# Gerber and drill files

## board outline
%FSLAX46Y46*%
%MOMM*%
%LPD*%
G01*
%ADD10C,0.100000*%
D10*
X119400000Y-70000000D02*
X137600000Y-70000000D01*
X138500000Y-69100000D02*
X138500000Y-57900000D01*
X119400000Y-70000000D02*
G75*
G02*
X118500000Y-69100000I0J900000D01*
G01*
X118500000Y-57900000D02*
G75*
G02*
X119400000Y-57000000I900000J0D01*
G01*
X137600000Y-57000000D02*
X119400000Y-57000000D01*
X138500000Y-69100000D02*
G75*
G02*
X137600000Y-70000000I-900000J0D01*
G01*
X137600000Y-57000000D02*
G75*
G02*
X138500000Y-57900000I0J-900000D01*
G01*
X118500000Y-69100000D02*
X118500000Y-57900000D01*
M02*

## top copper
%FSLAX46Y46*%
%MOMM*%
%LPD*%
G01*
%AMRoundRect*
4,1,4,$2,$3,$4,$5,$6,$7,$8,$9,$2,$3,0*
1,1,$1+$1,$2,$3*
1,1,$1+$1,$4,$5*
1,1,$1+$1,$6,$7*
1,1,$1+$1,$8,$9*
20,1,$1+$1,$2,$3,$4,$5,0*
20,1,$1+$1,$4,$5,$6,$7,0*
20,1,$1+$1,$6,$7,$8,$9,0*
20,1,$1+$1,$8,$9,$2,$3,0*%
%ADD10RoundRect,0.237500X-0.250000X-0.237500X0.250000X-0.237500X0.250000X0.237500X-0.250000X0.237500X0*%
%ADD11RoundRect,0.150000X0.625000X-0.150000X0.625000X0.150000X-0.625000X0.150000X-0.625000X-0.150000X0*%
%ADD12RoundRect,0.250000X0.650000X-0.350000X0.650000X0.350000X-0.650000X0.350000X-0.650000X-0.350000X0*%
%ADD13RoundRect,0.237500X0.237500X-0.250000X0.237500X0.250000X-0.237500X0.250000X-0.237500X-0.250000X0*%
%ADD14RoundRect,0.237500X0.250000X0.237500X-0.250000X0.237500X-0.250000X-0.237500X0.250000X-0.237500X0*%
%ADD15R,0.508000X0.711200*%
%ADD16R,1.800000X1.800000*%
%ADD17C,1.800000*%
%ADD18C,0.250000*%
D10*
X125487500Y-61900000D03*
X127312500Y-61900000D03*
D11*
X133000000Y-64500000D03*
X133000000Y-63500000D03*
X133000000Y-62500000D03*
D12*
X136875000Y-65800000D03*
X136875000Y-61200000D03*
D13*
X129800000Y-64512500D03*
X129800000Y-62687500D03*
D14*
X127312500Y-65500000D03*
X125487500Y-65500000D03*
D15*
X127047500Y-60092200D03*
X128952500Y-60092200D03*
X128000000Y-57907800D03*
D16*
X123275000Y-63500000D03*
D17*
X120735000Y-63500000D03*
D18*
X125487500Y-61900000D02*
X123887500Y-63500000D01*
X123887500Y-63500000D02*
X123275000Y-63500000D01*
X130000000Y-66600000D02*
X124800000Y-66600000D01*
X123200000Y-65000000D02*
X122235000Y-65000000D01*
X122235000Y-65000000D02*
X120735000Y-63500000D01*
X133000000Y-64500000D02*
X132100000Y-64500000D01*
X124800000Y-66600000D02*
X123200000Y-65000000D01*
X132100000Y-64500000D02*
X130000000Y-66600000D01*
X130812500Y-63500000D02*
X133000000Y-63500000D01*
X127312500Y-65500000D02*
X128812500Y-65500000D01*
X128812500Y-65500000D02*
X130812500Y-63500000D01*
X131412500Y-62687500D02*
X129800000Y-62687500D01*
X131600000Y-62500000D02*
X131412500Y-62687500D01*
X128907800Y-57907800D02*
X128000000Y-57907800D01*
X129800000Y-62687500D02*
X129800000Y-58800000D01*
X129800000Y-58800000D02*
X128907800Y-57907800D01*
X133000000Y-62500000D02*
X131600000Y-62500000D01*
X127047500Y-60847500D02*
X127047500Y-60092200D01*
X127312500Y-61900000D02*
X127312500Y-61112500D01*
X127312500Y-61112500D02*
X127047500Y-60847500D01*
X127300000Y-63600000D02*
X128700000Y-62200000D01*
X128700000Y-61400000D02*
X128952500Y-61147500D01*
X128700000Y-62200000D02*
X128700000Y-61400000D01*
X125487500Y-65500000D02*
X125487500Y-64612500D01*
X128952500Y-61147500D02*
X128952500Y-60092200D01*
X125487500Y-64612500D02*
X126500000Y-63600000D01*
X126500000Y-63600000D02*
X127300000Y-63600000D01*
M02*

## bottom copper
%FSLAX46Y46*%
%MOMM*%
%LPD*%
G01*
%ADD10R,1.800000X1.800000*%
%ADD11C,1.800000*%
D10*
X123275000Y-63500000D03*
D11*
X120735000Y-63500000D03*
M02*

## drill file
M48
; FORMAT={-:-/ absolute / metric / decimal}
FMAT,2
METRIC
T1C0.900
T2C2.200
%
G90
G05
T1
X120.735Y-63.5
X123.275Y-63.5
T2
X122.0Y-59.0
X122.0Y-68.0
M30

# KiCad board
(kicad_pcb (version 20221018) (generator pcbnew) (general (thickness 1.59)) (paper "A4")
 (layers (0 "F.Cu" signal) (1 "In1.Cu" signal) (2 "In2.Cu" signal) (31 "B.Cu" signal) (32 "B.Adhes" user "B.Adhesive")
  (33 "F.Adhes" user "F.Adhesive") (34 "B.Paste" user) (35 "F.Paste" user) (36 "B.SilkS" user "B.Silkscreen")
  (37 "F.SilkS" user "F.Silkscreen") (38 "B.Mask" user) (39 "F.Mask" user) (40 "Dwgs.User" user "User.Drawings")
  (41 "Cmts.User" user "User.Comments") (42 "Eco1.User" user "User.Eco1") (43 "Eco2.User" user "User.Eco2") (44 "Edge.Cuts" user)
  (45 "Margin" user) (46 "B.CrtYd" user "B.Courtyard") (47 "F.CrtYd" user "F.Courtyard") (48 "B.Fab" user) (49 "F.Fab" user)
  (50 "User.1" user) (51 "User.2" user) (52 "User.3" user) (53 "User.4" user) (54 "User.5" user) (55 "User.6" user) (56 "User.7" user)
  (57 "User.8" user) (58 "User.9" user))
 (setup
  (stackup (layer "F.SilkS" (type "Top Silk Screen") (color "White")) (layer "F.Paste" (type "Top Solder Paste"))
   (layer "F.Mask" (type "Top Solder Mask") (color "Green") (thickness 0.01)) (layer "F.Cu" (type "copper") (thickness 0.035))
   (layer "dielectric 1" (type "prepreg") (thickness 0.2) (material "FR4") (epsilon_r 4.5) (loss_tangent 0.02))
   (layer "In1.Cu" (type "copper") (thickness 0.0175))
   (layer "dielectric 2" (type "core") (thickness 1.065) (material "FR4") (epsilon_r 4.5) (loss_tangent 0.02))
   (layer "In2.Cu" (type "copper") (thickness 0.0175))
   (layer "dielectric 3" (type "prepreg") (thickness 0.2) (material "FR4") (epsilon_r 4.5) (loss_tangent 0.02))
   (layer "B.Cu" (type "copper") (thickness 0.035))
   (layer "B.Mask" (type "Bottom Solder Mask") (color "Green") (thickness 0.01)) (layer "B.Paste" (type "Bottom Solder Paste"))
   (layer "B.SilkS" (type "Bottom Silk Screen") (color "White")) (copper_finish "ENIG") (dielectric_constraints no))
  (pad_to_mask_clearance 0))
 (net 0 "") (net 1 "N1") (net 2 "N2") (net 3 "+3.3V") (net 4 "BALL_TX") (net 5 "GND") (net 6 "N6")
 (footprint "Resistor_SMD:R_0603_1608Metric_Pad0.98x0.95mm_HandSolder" (layer "F.Cu") (at 126.4 61.9)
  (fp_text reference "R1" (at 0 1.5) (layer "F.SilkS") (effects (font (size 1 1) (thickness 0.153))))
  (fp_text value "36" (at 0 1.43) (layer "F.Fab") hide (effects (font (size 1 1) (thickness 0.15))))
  (pad "1" smd roundrect (at -0.9125 0) (size 0.975 0.95) (layers "F.Cu" "F.Paste" "F.Mask") (roundrect_rratio 0.25) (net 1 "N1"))
  (pad "2" smd roundrect (at 0.9125 0) (size 0.975 0.95) (layers "F.Cu" "F.Paste" "F.Mask") (roundrect_rratio 0.25) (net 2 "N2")))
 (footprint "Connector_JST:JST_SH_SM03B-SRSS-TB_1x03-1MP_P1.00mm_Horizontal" (layer "F.Cu") (at 135 63.5 90)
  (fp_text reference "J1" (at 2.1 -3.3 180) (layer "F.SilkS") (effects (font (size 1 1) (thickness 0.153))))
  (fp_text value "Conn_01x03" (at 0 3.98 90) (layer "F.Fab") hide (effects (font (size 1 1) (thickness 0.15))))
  (pad "1" smd roundrect (at -1 -2 90) (size 0.6 1.55) (layers "F.Cu" "F.Paste" "F.Mask") (roundrect_rratio 0.25) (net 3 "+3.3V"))
  (pad "2" smd roundrect (at 0 -2 90) (size 0.6 1.55) (layers "F.Cu" "F.Paste" "F.Mask") (roundrect_rratio 0.25) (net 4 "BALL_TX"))
  (pad "3" smd roundrect (at 1 -2 90) (size 0.6 1.55) (layers "F.Cu" "F.Paste" "F.Mask") (roundrect_rratio 0.25) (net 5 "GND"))
  (pad "MP" smd roundrect (at -2.3 1.875 90) (size 1.2 1.8) (layers "F.Cu" "F.Paste" "F.Mask") (roundrect_rratio 0.208333))
  (pad "MP" smd roundrect (at 2.3 1.875 90) (size 1.2 1.8) (layers "F.Cu" "F.Paste" "F.Mask") (roundrect_rratio 0.208333)))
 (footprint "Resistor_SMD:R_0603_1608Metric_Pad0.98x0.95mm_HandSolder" (layer "F.Cu") (at 129.8 63.6 90)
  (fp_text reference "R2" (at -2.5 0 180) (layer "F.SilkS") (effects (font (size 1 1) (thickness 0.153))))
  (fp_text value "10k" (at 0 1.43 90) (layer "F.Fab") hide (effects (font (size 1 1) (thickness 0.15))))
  (pad "1" smd roundrect (at -0.9125 0 90) (size 0.975 0.95) (layers "F.Cu" "F.Paste" "F.Mask") (roundrect_rratio 0.25) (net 4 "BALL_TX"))
  (pad "2" smd roundrect (at 0.9125 0 90) (size 0.975 0.95) (layers "F.Cu" "F.Paste" "F.Mask") (roundrect_rratio 0.25) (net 5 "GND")))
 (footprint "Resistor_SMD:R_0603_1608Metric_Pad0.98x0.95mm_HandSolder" (layer "F.Cu") (at 126.4 65.5 180)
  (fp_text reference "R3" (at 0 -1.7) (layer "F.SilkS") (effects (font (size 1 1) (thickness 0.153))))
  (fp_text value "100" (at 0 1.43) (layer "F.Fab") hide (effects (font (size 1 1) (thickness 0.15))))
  (pad "1" smd roundrect (at -0.9125 0 180) (size 0.975 0.95) (layers "F.Cu" "F.Paste" "F.Mask") (roundrect_rratio 0.25) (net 4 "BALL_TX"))
  (pad "2" smd roundrect (at 0.9125 0 180) (size 0.975 0.95) (layers "F.Cu" "F.Paste" "F.Mask") (roundrect_rratio 0.25) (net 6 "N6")))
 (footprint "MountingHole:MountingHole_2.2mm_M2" (layer "F.Cu") (at 122 68 -90)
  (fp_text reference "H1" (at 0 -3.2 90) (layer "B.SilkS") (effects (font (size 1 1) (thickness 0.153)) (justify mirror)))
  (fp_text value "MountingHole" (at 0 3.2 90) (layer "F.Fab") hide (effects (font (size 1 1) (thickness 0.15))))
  (pad "" np_thru_hole circle (at 0 0 270) (size 2.2 2.2) (drill 2.2) (layers "*.Cu" "*.Mask")))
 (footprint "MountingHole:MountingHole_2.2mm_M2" (layer "F.Cu") (at 122 59 -90)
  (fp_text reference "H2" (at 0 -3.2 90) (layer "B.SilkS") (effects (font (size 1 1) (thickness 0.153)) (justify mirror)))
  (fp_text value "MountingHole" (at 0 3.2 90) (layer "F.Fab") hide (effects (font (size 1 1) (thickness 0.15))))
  (pad "" np_thru_hole circle (at 0 0 270) (size 2.2 2.2) (drill 2.2) (layers "*.Cu" "*.Mask")))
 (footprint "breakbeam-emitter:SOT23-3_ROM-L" (layer "F.Cu") (at 128 59)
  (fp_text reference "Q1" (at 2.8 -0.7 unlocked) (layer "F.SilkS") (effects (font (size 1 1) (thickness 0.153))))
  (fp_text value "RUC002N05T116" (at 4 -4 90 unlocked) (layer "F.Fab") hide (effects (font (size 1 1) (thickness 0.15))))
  (pad "1" smd rect (at -0.9525 1.0922) (size 0.508 0.7112) (layers "F.Cu" "F.Paste" "F.Mask") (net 2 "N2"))
  (pad "2" smd rect (at 0.9525 1.0922) (size 0.508 0.7112) (layers "F.Cu" "F.Paste" "F.Mask") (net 6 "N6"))
  (pad "3" smd rect (at 0 -1.0922) (size 0.508 0.7112) (layers "F.Cu" "F.Paste" "F.Mask") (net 5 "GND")))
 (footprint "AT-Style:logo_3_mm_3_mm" (layer "B.Cu") (at 135.5 60.5 180)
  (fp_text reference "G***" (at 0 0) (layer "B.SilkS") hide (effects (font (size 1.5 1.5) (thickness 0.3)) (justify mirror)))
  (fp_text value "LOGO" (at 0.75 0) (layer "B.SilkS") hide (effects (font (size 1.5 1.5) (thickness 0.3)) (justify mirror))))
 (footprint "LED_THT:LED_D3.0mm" (layer "B.Cu") (at 123.275 63.5 180)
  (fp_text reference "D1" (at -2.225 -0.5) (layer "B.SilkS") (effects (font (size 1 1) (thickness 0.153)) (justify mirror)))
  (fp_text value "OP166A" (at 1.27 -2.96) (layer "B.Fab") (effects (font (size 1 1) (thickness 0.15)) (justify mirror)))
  (pad "1" thru_hole rect (at 0 0 180) (size 1.8 1.8) (drill 0.9) (layers "*.Cu" "*.Mask") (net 1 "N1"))
  (pad "2" thru_hole circle (at 2.54 0 180) (size 1.8 1.8) (drill 0.9) (layers "*.Cu" "*.Mask") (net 3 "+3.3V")))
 (gr_line (start 119.4 70) (end 137.6 70) (stroke (width 0.1) (type default)) (layer "Edge.Cuts"))
 (gr_line (start 138.5 69.1) (end 138.5 57.9) (stroke (width 0.1) (type default)) (layer "Edge.Cuts"))
 (gr_arc (start 119.4 70) (mid 118.763604 69.736396) (end 118.5 69.1) (stroke (width 0.1) (type default)) (layer "Edge.Cuts"))
 (gr_arc (start 118.5 57.9) (mid 118.763604 57.263604) (end 119.4 57) (stroke (width 0.1) (type default)) (layer "Edge.Cuts"))
 (gr_line (start 137.6 57) (end 119.4 57) (stroke (width 0.1) (type default)) (layer "Edge.Cuts"))
 (gr_arc (start 138.5 69.1) (mid 138.236396 69.736396) (end 137.6 70) (stroke (width 0.1) (type default)) (layer "Edge.Cuts"))
 (gr_arc (start 137.6 57) (mid 138.236396 57.263604) (end 138.5 57.9) (stroke (width 0.1) (type default)) (layer "Edge.Cuts"))
 (gr_line (start 118.5 69.1) (end 118.5 57.9) (stroke (width 0.1) (type default)) (layer "Edge.Cuts"))
 (segment (start 125.4875 61.9) (end 123.8875 63.5) (width 0.25) (layer "F.Cu") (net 1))
 (segment (start 123.8875 63.5) (end 123.275 63.5) (width 0.25) (layer "F.Cu") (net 1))
 (segment (start 130 66.6) (end 124.8 66.6) (width 0.25) (layer "F.Cu") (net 3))
 (segment (start 123.2 65) (end 122.235 65) (width 0.25) (layer "F.Cu") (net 3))
 (segment (start 122.235 65) (end 120.735 63.5) (width 0.25) (layer "F.Cu") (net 3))
 (segment (start 133 64.5) (end 132.1 64.5) (width 0.25) (layer "F.Cu") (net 3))
 (segment (start 124.8 66.6) (end 123.2 65) (width 0.25) (layer "F.Cu") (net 3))
 (segment (start 132.1 64.5) (end 130 66.6) (width 0.25) (layer "F.Cu") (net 3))
 (segment (start 130.8125 63.5) (end 133 63.5) (width 0.25) (layer "F.Cu") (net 4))
 (segment (start 127.3125 65.5) (end 128.8125 65.5) (width 0.25) (layer "F.Cu") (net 4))
 (segment (start 128.8125 65.5) (end 130.8125 63.5) (width 0.25) (layer "F.Cu") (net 4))
 (segment (start 131.4125 62.6875) (end 129.8 62.6875) (width 0.25) (layer "F.Cu") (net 5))
 (segment (start 131.6 62.5) (end 131.4125 62.6875) (width 0.25) (layer "F.Cu") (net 5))
 (segment (start 128.9078 57.9078) (end 128 57.9078) (width 0.25) (layer "F.Cu") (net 5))
 (segment (start 129.8 62.6875) (end 129.8 58.8) (width 0.25) (layer "F.Cu") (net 5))
 (segment (start 129.8 58.8) (end 128.9078 57.9078) (width 0.25) (layer "F.Cu") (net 5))
 (segment (start 133 62.5) (end 131.6 62.5) (width 0.25) (layer "F.Cu") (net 5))
 (segment (start 127.0475 60.8475) (end 127.0475 60.0922) (width 0.25) (layer "F.Cu") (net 2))
 (segment (start 127.3125 61.9) (end 127.3125 61.1125) (width 0.25) (layer "F.Cu") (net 2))
 (segment (start 127.3125 61.1125) (end 127.0475 60.8475) (width 0.25) (layer "F.Cu") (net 2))
 (segment (start 127.3 63.6) (end 128.7 62.2) (width 0.25) (layer "F.Cu") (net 6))
 (segment (start 128.7 61.4) (end 128.9525 61.1475) (width 0.25) (layer "F.Cu") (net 6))
 (segment (start 128.7 62.2) (end 128.7 61.4) (width 0.25) (layer "F.Cu") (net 6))
 (segment (start 125.4875 65.5) (end 125.4875 64.6125) (width 0.25) (layer "F.Cu") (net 6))
 (segment (start 128.9525 61.1475) (end 128.9525 60.0922) (width 0.25) (layer "F.Cu") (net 6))
 (segment (start 125.4875 64.6125) (end 126.5 63.6) (width 0.25) (layer "F.Cu") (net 6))
 (segment (start 126.5 63.6) (end 127.3 63.6) (width 0.25) (layer "F.Cu") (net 6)))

